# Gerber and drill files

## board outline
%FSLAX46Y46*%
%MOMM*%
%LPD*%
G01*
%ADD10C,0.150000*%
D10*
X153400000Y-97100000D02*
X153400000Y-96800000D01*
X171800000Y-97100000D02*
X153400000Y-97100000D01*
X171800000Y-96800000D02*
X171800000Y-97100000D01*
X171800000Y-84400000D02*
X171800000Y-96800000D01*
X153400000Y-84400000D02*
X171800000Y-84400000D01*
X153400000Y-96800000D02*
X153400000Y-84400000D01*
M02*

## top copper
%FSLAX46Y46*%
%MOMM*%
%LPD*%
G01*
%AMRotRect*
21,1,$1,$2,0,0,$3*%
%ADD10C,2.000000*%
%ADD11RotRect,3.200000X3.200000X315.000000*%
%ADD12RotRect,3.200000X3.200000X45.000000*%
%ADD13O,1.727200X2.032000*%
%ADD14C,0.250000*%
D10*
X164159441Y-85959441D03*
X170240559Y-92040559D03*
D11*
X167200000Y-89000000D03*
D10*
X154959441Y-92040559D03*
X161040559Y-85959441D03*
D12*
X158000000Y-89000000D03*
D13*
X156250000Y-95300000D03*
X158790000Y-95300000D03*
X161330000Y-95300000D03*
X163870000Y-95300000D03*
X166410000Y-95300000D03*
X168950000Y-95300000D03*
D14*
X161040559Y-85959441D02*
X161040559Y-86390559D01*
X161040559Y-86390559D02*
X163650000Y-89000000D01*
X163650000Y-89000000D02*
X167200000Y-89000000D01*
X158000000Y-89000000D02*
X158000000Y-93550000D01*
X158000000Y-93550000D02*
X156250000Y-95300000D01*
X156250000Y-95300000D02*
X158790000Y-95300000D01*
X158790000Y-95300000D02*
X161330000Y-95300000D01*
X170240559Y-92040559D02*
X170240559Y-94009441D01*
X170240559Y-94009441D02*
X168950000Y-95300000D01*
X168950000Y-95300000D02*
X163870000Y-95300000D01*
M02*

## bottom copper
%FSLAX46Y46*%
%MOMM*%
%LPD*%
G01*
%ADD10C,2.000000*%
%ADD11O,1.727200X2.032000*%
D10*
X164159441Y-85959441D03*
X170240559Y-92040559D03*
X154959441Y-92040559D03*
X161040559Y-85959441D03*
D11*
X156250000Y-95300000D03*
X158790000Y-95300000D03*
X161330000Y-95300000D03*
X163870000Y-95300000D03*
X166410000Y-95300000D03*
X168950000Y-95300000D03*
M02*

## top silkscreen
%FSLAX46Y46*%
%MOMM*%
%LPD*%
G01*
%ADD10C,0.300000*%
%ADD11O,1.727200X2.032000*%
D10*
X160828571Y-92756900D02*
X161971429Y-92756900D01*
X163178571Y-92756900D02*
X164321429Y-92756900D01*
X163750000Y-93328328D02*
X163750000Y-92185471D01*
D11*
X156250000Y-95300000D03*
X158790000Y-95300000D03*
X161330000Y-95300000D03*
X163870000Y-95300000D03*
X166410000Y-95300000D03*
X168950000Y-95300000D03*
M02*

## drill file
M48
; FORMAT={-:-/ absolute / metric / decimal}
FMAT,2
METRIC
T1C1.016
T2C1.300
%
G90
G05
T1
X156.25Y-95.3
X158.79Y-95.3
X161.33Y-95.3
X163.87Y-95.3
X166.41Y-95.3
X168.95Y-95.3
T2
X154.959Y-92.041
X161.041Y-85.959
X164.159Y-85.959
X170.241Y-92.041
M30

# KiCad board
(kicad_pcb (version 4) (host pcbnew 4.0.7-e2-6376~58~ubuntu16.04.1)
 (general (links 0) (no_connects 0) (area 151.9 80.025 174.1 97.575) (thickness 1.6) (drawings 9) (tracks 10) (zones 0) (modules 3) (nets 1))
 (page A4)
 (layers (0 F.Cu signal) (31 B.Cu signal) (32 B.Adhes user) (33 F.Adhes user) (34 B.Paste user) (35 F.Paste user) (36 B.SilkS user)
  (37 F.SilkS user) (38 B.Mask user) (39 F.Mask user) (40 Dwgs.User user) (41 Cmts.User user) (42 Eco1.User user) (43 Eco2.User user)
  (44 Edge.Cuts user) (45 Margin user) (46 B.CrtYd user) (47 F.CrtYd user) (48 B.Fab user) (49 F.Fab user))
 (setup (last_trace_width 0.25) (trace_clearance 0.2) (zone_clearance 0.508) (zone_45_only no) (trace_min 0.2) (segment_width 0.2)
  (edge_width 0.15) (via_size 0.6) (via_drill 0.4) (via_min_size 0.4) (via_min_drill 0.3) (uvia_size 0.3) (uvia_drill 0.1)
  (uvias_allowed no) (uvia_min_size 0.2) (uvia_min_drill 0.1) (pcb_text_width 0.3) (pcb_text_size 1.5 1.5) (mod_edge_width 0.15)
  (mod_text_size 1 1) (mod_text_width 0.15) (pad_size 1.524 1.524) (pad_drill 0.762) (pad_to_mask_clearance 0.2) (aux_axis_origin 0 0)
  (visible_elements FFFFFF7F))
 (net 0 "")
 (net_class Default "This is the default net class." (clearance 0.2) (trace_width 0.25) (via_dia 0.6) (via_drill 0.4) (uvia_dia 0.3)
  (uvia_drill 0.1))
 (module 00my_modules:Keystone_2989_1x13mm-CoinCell (layer F.Cu) (at 167.2 89 315)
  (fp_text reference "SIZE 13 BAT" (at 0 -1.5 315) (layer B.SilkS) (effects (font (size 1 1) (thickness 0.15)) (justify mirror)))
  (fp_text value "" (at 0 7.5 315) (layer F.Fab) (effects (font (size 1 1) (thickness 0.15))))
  (pad 1 thru_hole circle (at -4.3 0 315) (size 2 2) (drill 1.3) (layers *.Cu *.Mask))
  (pad 1 thru_hole circle (at 4.3 0 315) (size 2 2) (drill 1.3) (layers *.Cu *.Mask))
  (pad 2 smd rect (at 0 0 315) (size 3.2 3.2) (layers F.Cu F.Mask)))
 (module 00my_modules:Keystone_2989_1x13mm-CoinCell (layer F.Cu) (at 158 89 45)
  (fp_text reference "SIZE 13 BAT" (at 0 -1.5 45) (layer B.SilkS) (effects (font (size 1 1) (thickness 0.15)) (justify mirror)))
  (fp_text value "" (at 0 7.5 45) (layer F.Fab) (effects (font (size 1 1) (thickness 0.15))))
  (pad 1 thru_hole circle (at -4.3 0 45) (size 2 2) (drill 1.3) (layers *.Cu *.Mask))
  (pad 1 thru_hole circle (at 4.3 0 45) (size 2 2) (drill 1.3) (layers *.Cu *.Mask))
  (pad 2 smd rect (at 0 0 45) (size 3.2 3.2) (layers F.Cu F.Mask)))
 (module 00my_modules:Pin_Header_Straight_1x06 (layer F.Cu) (at 156.25 95.3 90)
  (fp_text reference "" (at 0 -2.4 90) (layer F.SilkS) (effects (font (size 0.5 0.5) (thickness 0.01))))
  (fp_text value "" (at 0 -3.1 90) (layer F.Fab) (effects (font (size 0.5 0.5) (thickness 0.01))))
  (pad 1 thru_hole oval (at 0 0 90) (size 2.032 1.7272) (drill 1.016) (layers *.Cu *.Mask F.SilkS))
  (pad 2 thru_hole oval (at 0 2.54 90) (size 2.032 1.7272) (drill 1.016) (layers *.Cu *.Mask F.SilkS))
  (pad 3 thru_hole oval (at 0 5.08 90) (size 2.032 1.7272) (drill 1.016) (layers *.Cu *.Mask F.SilkS))
  (pad 4 thru_hole oval (at 0 7.62 90) (size 2.032 1.7272) (drill 1.016) (layers *.Cu *.Mask F.SilkS))
  (pad 5 thru_hole oval (at 0 10.16 90) (size 2.032 1.7272) (drill 1.016) (layers *.Cu *.Mask F.SilkS))
  (pad 6 thru_hole oval (at 0 12.7 90) (size 2.032 1.7272) (drill 1.016) (layers *.Cu *.Mask F.SilkS)))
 (gr_line (start 153.4 97.1) (end 153.4 96.8) (angle 90) (layer Edge.Cuts) (width 0.15))
 (gr_line (start 171.8 97.1) (end 153.4 97.1) (angle 90) (layer Edge.Cuts) (width 0.15))
 (gr_line (start 171.8 96.8) (end 171.8 97.1) (angle 90) (layer Edge.Cuts) (width 0.15))
 (gr_line (start 171.8 84.4) (end 171.8 96.8) (angle 90) (layer Edge.Cuts) (width 0.15))
 (gr_line (start 153.4 84.4) (end 171.8 84.4) (angle 90) (layer Edge.Cuts) (width 0.15))
 (gr_line (start 153.4 96.8) (end 153.4 84.4) (angle 90) (layer Edge.Cuts) (width 0.15))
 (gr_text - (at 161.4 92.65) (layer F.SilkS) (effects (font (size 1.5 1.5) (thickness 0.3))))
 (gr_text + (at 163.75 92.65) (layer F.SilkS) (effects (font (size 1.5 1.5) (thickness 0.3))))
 (segment (start 161.040559 85.959441) (end 161.040559 86.390559) (width 0.25) (layer F.Cu) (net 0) (status C00000))
 (segment (start 161.040559 86.390559) (end 163.65 89) (width 0.25) (layer F.Cu) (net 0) (status 400000))
 (segment (start 163.65 89) (end 167.2 89) (width 0.25) (layer F.Cu) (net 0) (status 800000))
 (segment (start 158 89) (end 158 93.55) (width 0.25) (layer F.Cu) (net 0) (status 400000))
 (segment (start 158 93.55) (end 156.25 95.3) (width 0.25) (layer F.Cu) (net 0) (status 800000))
 (segment (start 156.25 95.3) (end 158.79 95.3) (width 0.25) (layer F.Cu) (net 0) (status C00000))
 (segment (start 158.79 95.3) (end 161.33 95.3) (width 0.25) (layer F.Cu) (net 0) (status C00000))
 (segment (start 170.240559 92.040559) (end 170.240559 94.009441) (width 0.25) (layer F.Cu) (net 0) (status 400000))
 (segment (start 170.240559 94.009441) (end 168.95 95.3) (width 0.25) (layer F.Cu) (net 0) (status 800000))
 (segment (start 168.95 95.3) (end 163.87 95.3) (width 0.25) (layer F.Cu) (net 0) (status C00000)))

